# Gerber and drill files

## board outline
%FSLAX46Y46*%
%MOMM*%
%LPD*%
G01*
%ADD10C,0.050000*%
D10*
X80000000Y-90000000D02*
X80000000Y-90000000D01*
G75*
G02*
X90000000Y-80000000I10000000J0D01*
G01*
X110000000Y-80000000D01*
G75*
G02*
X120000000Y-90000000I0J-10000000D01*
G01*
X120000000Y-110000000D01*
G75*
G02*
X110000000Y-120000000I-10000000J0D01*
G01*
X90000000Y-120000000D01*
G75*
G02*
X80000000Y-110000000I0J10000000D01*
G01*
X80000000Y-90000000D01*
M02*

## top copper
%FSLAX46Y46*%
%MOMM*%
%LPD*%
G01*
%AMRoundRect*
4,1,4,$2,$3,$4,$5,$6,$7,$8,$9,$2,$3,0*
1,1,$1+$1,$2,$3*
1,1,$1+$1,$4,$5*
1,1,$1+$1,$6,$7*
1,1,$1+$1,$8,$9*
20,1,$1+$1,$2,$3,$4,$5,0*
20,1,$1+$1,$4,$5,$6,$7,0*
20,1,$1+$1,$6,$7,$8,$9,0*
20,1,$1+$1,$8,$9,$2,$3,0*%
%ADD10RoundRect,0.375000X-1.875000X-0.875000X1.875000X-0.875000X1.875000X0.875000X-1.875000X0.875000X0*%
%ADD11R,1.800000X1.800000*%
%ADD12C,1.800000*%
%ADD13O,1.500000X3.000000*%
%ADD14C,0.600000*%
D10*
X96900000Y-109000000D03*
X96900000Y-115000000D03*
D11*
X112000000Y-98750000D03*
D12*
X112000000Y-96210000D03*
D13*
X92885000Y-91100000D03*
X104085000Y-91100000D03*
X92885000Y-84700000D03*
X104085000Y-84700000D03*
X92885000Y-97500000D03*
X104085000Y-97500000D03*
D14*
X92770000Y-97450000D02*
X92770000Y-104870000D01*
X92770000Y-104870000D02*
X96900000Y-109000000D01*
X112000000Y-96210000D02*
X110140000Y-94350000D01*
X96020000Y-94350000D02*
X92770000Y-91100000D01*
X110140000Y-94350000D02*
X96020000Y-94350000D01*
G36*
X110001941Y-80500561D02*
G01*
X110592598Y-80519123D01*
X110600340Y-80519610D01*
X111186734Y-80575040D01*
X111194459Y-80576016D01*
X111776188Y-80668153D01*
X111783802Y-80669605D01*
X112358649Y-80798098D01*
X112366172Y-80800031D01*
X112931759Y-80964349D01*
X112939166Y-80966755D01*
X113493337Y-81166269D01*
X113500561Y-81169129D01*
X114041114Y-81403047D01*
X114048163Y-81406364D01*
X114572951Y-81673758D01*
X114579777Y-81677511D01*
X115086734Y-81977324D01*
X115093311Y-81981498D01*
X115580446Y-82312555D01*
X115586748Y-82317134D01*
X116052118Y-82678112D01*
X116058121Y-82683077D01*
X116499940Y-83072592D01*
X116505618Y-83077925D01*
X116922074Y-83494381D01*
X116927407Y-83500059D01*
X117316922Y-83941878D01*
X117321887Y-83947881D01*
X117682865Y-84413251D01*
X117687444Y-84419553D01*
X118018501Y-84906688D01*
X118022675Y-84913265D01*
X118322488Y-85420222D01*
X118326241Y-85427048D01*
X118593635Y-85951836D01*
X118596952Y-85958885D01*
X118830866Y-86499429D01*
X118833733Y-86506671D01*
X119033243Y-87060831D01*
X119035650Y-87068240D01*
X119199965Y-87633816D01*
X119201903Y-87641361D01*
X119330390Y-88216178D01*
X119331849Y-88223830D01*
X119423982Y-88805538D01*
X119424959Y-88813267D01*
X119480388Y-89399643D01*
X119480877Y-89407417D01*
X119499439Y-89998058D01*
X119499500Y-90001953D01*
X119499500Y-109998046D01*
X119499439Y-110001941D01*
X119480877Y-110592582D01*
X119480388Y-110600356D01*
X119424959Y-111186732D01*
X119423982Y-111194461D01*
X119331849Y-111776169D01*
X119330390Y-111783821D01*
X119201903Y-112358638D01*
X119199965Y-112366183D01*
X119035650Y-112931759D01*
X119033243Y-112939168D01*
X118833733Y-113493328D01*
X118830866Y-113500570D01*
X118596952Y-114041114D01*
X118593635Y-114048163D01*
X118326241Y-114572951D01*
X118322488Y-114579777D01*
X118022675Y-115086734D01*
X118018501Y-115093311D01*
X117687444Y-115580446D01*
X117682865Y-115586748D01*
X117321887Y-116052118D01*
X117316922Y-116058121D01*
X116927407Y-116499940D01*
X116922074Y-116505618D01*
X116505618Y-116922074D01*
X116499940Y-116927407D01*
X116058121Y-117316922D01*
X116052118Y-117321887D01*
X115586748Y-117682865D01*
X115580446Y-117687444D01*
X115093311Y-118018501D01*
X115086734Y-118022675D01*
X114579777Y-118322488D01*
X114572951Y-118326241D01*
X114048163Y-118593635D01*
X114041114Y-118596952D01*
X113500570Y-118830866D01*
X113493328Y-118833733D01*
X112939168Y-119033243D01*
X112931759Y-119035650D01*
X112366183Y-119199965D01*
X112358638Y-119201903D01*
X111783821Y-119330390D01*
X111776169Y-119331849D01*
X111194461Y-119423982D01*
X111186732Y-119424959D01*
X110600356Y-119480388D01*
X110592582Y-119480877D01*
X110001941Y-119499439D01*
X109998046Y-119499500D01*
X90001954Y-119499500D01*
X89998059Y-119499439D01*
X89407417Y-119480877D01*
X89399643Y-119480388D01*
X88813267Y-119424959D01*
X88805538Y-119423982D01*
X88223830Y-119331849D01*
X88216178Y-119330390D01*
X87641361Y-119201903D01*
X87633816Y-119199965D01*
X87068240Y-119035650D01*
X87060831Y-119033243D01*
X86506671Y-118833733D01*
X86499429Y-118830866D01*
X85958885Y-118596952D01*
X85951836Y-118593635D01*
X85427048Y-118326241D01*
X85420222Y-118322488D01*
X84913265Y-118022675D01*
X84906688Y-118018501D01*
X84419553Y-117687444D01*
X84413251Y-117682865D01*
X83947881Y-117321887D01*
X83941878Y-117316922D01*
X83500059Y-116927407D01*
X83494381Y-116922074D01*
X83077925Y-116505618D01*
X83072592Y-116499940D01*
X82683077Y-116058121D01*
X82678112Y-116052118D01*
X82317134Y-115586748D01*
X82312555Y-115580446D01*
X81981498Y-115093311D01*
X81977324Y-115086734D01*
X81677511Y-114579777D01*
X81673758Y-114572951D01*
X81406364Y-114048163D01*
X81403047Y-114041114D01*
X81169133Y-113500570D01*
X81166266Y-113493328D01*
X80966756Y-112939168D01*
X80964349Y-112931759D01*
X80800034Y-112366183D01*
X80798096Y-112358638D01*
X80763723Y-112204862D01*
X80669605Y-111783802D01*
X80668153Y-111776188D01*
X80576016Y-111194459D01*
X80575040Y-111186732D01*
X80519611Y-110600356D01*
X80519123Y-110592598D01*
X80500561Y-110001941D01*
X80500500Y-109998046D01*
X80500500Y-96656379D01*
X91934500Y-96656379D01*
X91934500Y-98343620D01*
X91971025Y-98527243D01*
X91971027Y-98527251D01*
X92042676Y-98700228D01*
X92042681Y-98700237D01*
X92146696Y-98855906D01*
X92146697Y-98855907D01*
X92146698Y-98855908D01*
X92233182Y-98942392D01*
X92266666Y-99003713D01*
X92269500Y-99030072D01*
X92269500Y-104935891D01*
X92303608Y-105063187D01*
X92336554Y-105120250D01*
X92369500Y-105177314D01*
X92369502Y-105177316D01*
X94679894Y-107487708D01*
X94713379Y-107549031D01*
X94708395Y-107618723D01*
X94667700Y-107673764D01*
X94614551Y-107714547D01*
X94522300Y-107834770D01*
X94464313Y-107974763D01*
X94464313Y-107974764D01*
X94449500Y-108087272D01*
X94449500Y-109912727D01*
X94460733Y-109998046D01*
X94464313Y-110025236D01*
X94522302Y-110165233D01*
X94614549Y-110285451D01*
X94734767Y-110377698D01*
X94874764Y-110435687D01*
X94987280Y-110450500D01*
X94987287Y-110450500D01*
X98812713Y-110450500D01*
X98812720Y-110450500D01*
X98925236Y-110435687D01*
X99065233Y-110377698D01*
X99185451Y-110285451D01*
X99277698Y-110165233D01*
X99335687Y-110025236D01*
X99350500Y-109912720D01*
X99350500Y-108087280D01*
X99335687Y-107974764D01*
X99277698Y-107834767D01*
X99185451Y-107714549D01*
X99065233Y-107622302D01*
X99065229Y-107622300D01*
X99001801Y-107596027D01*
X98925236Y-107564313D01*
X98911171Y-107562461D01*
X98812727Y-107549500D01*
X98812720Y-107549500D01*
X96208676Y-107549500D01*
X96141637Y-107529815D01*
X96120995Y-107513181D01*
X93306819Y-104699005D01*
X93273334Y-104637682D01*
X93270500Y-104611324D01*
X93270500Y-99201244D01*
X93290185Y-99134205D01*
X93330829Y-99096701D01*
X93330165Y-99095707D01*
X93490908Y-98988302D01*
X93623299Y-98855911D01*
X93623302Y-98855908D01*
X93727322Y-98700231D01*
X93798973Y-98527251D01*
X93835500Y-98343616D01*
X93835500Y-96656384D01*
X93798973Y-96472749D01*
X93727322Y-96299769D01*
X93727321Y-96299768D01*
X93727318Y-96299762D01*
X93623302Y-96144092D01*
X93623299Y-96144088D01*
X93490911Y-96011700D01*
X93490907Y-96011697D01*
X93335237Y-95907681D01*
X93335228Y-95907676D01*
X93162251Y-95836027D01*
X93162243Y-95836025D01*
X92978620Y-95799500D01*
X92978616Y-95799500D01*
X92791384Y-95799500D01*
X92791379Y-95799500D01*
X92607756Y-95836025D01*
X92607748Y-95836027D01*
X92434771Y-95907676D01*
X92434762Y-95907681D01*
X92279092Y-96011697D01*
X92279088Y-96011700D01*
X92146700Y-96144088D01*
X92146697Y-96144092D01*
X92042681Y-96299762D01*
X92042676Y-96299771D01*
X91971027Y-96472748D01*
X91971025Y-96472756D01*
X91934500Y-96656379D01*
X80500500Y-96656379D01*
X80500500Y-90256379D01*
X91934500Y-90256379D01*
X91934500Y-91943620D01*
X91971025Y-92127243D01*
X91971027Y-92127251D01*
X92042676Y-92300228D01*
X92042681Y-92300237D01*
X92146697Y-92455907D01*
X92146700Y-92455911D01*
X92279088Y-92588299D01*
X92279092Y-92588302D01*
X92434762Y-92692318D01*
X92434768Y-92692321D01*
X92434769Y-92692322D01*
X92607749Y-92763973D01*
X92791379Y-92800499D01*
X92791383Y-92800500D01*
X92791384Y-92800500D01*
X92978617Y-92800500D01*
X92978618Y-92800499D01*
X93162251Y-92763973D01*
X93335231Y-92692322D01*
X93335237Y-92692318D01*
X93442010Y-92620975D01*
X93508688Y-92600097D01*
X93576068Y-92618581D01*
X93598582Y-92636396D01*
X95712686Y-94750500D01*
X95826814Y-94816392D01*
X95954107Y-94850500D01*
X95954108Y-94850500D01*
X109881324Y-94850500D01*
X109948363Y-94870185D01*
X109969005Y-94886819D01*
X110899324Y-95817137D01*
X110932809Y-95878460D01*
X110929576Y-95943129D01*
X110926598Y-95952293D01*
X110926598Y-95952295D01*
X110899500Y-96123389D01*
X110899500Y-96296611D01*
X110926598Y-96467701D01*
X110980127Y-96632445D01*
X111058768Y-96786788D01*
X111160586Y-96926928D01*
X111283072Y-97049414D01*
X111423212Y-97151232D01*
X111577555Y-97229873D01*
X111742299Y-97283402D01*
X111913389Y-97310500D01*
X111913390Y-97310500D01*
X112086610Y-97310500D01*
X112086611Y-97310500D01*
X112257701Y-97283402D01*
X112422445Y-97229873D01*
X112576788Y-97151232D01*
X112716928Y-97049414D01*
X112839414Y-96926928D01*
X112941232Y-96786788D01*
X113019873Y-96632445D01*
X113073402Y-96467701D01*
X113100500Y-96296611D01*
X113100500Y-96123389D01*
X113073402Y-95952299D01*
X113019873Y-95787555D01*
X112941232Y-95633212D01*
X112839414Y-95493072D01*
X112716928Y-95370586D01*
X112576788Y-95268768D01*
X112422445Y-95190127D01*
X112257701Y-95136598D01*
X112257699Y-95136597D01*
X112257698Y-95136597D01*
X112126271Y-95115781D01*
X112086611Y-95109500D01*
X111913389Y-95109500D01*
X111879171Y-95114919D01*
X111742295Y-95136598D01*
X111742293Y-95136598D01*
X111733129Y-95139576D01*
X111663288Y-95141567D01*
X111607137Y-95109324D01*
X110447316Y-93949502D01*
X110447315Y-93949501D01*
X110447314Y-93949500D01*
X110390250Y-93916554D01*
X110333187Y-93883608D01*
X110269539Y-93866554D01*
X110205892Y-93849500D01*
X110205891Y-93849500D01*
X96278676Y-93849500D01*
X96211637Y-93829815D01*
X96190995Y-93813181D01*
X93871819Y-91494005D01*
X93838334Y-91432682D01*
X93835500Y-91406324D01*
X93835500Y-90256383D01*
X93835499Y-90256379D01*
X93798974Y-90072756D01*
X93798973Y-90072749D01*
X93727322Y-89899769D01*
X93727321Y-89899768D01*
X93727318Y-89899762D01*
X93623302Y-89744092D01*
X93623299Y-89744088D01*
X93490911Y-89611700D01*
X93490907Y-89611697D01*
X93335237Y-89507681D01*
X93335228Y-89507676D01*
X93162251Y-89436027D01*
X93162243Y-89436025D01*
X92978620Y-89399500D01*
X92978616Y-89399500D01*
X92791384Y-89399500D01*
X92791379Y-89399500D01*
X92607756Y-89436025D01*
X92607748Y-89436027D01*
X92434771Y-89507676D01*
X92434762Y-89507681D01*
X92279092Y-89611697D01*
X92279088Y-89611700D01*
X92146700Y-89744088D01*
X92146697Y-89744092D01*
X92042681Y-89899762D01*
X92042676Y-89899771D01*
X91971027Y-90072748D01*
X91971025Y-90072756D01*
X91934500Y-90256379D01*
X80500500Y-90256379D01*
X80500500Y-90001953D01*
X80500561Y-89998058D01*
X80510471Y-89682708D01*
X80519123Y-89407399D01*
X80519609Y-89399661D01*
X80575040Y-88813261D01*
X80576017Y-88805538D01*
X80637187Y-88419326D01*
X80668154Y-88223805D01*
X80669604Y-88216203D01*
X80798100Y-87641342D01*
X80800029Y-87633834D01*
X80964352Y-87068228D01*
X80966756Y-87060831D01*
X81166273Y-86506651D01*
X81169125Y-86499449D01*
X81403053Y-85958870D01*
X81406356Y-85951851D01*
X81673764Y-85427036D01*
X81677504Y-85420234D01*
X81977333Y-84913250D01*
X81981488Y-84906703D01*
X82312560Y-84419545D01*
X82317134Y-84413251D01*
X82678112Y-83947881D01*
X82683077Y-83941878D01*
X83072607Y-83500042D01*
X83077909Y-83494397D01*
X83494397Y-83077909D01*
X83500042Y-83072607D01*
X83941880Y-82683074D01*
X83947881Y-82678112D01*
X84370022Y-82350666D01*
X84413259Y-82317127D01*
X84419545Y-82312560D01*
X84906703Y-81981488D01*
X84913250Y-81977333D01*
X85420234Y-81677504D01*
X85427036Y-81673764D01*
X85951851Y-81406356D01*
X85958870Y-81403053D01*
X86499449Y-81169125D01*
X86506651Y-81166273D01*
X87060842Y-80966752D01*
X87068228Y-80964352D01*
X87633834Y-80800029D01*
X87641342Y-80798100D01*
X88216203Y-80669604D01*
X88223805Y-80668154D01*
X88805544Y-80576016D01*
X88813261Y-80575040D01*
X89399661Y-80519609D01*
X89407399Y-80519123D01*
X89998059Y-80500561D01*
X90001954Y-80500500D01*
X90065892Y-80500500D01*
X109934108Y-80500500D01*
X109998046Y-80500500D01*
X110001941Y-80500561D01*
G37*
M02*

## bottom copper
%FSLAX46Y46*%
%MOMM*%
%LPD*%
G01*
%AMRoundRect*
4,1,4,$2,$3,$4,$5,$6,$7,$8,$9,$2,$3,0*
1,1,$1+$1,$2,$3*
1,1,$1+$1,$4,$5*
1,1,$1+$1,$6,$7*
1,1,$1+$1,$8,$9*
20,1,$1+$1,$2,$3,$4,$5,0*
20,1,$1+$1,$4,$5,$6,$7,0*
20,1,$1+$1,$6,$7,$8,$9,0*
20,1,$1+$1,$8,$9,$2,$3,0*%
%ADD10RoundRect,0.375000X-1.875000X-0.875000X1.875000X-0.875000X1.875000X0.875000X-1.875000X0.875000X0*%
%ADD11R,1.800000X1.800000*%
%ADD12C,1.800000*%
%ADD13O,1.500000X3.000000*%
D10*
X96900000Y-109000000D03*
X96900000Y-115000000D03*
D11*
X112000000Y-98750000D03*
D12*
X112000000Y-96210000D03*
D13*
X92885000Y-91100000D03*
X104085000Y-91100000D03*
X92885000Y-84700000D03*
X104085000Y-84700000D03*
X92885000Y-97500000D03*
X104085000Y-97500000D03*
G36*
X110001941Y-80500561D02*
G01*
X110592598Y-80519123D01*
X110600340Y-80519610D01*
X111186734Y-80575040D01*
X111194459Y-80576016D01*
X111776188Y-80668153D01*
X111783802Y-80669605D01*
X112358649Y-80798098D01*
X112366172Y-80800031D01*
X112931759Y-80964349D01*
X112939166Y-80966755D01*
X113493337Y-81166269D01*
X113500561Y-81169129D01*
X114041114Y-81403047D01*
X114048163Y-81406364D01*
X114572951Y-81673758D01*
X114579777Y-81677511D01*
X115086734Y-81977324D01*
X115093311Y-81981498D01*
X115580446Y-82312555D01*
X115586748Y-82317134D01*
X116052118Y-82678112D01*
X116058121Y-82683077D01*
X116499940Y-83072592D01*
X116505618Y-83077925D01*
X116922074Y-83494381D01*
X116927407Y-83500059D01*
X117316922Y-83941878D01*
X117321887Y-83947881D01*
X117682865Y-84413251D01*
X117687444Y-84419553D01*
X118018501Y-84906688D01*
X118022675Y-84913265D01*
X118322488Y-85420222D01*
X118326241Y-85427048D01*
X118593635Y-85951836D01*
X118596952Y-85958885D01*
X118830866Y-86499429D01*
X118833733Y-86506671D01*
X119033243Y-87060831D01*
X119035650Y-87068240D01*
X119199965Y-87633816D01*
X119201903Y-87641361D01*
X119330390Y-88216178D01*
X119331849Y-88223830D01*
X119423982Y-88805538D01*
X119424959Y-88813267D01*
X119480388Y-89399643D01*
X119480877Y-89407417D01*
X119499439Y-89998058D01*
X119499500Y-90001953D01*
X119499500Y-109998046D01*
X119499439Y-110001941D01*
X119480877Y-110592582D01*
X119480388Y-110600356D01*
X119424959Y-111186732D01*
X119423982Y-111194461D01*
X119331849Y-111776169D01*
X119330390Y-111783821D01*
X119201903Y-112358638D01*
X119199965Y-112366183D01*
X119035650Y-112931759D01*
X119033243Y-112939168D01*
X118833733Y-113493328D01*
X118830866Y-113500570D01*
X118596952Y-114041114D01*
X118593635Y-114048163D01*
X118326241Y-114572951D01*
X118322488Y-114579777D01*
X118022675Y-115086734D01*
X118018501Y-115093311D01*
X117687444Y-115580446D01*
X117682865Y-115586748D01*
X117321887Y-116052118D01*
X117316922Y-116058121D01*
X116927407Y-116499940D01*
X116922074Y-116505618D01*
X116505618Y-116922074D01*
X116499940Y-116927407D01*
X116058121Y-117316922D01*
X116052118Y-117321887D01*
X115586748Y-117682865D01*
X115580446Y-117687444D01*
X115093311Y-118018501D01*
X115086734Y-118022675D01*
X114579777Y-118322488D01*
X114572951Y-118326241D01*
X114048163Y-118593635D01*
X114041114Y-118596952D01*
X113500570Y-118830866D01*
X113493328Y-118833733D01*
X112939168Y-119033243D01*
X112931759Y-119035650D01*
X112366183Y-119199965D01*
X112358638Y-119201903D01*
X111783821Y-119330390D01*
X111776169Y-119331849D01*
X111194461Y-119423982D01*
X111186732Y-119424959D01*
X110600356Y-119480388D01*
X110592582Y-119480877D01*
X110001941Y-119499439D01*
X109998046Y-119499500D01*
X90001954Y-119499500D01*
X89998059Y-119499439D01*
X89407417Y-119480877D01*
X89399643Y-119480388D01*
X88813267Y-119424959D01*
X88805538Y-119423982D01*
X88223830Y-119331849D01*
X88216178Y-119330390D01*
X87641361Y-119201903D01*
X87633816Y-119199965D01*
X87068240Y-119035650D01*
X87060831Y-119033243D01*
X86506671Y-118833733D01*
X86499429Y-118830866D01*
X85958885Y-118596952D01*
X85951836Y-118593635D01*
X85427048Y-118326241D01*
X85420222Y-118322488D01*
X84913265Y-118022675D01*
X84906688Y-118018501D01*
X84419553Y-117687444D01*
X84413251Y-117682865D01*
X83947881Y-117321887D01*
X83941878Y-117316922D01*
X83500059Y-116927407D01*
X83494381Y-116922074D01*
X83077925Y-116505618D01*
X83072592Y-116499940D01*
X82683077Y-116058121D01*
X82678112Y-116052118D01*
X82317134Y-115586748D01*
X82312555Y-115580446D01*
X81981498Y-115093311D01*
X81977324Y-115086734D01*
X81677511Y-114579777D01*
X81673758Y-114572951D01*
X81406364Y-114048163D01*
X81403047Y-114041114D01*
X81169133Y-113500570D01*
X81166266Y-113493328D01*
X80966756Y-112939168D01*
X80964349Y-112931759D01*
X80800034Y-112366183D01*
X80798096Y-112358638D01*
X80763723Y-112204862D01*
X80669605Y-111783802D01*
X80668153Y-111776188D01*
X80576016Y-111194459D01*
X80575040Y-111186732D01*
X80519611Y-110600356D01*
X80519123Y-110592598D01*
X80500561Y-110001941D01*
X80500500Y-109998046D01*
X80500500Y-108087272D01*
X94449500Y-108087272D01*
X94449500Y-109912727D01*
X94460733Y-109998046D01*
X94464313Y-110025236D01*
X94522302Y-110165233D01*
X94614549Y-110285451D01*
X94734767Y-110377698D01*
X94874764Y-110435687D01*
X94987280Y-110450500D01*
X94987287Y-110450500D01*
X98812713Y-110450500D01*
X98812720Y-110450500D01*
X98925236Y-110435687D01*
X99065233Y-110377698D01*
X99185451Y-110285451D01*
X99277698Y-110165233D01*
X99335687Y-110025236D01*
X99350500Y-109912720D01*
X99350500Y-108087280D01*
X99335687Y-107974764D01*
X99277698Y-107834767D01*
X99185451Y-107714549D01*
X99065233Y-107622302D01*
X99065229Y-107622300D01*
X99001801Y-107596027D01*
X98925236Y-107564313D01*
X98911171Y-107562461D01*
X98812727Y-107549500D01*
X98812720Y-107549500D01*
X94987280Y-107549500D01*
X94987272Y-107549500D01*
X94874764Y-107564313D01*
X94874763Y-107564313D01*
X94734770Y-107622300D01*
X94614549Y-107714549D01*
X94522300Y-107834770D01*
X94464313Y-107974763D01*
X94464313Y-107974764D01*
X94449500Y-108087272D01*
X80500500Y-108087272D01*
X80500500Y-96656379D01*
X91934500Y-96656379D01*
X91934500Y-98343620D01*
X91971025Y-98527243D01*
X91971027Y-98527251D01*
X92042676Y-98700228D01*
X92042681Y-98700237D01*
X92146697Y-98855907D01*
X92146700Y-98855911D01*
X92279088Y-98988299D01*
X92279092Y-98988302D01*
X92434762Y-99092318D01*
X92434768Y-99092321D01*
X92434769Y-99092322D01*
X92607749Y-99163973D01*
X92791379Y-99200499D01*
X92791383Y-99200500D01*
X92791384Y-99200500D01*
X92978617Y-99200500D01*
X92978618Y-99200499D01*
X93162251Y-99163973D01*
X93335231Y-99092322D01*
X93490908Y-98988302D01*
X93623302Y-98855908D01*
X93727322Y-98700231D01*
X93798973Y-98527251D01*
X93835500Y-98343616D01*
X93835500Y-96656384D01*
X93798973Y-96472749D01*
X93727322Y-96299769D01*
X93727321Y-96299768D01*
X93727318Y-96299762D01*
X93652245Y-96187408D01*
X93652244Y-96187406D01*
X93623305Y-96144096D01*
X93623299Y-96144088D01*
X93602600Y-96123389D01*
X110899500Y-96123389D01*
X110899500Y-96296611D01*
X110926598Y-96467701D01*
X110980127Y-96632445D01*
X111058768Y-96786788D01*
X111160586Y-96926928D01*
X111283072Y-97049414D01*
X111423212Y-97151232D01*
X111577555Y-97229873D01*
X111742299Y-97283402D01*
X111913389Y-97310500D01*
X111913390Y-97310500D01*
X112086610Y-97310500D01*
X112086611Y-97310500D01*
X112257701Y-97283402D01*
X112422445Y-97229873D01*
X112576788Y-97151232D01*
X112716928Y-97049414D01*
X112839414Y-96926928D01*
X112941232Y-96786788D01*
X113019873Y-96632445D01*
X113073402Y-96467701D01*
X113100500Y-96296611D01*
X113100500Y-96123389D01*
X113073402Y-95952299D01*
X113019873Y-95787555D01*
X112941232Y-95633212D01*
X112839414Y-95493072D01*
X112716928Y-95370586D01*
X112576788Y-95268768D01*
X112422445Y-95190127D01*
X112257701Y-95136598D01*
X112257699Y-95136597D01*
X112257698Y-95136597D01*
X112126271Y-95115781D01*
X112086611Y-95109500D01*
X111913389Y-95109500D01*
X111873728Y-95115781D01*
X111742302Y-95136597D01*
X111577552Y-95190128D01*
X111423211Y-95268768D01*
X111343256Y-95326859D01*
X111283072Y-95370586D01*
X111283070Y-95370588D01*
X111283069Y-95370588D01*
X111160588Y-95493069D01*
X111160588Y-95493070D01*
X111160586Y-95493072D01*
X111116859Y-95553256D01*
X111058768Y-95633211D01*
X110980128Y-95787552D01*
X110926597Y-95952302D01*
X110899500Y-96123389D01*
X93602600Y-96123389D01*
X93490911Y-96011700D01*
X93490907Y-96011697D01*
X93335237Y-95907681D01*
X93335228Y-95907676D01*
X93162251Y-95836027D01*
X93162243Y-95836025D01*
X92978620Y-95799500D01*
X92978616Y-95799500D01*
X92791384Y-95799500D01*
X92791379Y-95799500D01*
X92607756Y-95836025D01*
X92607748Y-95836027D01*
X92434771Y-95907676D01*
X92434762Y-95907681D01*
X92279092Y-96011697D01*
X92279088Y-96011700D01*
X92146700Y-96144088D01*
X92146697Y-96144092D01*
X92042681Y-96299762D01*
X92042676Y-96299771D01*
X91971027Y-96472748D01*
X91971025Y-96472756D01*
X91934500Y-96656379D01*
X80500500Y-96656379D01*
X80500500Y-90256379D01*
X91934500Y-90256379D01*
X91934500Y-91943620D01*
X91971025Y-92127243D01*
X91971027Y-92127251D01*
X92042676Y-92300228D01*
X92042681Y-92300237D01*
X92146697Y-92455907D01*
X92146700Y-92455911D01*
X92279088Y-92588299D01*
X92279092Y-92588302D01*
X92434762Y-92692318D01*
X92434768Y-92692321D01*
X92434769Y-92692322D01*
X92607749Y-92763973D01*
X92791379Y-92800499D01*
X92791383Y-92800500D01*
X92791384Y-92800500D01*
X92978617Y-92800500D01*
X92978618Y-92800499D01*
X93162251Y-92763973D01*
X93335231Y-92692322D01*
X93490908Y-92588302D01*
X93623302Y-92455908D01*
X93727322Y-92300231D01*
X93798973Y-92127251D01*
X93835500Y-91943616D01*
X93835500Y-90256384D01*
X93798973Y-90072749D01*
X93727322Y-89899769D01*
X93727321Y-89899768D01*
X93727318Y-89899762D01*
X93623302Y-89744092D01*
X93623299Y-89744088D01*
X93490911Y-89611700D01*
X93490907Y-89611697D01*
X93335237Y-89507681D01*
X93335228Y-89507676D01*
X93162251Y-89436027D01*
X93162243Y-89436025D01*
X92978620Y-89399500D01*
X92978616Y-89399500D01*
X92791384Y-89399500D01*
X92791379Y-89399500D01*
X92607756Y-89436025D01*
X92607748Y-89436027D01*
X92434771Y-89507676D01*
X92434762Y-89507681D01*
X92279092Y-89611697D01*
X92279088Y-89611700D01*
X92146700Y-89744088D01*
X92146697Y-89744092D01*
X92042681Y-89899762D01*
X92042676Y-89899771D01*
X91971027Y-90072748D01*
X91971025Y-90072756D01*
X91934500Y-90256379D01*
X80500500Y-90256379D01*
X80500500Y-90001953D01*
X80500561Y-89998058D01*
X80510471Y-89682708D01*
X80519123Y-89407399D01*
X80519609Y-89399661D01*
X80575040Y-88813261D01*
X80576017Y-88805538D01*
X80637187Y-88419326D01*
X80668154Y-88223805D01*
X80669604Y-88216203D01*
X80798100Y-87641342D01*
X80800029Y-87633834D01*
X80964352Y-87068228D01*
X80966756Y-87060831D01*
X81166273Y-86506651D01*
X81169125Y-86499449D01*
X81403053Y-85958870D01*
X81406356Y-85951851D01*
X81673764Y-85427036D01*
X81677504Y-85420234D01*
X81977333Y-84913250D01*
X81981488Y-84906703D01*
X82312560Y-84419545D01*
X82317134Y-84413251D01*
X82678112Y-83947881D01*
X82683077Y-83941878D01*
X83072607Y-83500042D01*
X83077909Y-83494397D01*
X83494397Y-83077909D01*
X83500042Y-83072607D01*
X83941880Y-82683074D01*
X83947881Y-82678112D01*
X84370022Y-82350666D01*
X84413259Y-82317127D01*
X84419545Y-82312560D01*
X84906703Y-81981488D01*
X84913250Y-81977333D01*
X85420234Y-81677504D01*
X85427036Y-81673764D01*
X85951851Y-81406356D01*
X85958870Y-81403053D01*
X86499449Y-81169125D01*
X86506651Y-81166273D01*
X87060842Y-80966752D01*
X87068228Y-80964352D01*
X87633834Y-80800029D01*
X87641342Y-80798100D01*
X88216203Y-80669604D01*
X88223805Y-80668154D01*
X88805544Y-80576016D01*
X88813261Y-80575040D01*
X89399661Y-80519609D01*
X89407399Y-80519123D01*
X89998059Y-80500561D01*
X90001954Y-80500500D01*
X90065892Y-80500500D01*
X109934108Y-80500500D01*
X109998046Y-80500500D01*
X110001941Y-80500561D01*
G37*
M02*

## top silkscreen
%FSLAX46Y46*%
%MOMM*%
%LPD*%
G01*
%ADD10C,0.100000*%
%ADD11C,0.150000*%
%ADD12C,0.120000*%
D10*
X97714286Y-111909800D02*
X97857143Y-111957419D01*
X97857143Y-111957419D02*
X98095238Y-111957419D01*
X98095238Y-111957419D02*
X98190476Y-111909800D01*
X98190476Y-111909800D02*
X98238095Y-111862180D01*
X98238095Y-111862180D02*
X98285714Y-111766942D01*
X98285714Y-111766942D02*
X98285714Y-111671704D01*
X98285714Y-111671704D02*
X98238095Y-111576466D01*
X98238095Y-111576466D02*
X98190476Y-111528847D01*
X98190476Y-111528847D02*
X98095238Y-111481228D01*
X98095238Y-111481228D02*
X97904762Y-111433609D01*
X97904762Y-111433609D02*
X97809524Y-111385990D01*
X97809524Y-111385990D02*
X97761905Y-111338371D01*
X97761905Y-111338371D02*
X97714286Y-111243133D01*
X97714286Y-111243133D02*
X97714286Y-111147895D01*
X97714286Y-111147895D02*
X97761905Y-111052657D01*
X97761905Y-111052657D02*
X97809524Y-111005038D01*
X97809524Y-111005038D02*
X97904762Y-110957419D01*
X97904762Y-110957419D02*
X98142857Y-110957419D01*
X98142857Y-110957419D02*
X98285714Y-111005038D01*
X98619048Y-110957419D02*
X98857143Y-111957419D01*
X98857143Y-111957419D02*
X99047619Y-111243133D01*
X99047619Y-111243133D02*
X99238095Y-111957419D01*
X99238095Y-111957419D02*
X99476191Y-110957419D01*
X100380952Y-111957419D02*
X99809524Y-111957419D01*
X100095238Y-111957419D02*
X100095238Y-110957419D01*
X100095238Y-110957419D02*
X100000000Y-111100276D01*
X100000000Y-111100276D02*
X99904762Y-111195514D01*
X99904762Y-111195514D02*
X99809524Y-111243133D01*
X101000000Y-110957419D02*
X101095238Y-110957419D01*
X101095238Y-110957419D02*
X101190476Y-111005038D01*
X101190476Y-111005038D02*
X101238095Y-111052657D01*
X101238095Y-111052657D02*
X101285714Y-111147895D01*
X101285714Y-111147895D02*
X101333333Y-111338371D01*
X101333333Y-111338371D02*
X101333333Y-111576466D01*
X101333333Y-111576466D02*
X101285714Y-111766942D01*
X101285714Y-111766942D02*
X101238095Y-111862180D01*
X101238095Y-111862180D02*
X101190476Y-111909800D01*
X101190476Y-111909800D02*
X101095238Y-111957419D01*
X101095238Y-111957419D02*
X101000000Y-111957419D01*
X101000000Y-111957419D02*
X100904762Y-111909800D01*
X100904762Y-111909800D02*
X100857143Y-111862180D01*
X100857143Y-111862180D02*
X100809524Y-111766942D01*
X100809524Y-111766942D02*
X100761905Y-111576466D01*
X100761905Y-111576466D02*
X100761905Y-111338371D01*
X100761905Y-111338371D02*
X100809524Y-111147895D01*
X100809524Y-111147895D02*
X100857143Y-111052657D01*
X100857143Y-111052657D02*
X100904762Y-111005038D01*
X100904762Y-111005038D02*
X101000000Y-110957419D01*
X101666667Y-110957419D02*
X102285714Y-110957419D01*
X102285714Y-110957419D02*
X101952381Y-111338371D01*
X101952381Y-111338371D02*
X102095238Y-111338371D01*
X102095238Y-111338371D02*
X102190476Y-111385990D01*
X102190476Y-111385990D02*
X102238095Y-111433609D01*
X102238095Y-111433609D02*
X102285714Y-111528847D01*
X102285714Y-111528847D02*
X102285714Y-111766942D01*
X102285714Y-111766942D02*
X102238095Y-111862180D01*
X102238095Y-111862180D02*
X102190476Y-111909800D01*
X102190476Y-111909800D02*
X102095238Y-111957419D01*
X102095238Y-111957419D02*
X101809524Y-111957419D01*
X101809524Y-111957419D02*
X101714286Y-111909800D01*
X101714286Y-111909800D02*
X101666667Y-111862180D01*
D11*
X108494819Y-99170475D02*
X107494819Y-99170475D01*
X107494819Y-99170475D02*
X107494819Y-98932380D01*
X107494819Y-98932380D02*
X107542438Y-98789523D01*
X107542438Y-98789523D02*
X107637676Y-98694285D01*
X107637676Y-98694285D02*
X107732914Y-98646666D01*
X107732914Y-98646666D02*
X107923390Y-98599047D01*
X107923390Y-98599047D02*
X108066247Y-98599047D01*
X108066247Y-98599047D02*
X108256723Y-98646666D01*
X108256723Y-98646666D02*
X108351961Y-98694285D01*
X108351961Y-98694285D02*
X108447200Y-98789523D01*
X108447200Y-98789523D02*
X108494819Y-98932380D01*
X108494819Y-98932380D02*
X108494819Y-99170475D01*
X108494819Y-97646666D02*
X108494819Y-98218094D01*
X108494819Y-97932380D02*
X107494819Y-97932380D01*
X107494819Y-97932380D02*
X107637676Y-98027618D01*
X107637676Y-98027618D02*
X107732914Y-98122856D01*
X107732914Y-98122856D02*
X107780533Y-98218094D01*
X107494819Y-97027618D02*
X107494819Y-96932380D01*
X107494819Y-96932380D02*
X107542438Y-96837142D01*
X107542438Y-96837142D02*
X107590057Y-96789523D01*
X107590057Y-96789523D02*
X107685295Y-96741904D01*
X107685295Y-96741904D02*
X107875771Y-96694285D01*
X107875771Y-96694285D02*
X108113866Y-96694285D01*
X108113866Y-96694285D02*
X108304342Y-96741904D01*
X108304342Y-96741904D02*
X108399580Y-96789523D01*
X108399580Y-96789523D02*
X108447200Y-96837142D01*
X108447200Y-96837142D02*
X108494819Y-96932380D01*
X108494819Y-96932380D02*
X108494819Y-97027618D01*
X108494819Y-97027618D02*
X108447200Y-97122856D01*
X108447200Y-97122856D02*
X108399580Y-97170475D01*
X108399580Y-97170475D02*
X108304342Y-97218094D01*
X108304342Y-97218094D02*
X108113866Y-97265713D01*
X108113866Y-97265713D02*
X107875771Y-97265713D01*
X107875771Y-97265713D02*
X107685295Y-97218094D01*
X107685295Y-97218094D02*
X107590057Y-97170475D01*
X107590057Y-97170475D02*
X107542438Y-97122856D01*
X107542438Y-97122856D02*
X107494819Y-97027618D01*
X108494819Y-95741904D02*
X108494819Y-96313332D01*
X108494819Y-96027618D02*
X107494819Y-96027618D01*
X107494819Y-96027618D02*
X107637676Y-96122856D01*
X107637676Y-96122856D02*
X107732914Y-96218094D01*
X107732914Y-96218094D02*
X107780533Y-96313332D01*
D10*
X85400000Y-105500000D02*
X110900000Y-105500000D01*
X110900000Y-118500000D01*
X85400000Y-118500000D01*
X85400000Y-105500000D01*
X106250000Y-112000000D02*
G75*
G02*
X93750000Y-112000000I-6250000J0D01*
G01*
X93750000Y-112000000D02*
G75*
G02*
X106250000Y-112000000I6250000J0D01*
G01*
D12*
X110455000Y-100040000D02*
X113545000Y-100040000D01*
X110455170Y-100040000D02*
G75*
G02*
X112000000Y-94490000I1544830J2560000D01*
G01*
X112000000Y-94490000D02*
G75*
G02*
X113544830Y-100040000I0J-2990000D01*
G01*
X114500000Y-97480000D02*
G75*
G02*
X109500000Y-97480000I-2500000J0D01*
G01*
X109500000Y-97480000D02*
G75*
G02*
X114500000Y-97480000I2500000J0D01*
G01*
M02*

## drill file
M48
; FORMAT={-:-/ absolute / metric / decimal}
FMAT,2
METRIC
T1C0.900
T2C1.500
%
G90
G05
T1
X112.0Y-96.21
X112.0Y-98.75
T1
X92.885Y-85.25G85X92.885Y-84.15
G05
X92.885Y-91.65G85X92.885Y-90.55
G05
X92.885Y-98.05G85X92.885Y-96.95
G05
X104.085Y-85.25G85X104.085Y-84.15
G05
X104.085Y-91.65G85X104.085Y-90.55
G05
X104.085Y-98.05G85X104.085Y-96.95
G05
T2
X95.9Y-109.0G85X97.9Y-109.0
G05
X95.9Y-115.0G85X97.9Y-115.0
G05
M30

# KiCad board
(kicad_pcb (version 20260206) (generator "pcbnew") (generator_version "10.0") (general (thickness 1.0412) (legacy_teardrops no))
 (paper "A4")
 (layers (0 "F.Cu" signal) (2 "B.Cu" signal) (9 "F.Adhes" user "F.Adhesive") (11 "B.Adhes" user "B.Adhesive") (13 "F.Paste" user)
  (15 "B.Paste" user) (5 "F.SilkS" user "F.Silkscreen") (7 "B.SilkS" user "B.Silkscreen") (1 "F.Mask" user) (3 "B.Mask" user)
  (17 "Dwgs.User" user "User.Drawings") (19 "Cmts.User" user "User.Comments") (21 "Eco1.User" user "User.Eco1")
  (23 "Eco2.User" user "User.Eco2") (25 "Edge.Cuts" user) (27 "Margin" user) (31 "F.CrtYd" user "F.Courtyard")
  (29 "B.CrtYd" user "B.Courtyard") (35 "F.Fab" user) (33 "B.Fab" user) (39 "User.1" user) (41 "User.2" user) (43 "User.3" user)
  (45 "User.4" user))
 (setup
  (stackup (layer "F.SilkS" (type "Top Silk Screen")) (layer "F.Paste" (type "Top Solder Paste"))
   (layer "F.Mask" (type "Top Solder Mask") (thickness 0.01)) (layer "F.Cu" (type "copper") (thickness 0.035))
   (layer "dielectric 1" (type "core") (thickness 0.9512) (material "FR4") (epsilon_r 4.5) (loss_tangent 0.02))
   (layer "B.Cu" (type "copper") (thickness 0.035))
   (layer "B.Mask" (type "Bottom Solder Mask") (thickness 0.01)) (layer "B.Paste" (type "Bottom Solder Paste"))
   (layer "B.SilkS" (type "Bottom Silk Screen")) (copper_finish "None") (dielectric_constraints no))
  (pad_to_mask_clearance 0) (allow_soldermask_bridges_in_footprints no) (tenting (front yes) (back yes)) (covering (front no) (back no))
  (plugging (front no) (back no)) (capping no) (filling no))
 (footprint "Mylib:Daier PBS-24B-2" (layer "F.Cu") (at 100 112)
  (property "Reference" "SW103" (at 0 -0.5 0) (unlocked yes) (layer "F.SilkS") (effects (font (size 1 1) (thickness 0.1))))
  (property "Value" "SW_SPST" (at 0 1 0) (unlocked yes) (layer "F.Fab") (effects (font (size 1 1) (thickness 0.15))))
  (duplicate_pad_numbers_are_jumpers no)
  (fp_rect (start -14.6 -6.5) (end 10.9 6.5) (stroke (width 0.1) (type solid)) (fill no) (layer "F.SilkS"))
  (fp_circle (center 0 0) (end 6.25 0) (stroke (width 0.1) (type solid)) (fill no) (layer "F.SilkS"))
  (pad "1" thru_hole roundrect (at -3.1 -3) (size 4.5 2.5) (drill oval 3.5 1.5) (layers "*.Cu" "*.Mask") (remove_unused_layers no)
   (roundrect_rratio 0.15) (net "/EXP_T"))
  (pad "2" thru_hole roundrect (at -3.1 3) (size 4.5 2.5) (drill oval 3.5 1.5) (layers "*.Cu" "*.Mask") (remove_unused_layers no)
   (roundrect_rratio 0.15) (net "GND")))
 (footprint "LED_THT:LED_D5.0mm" (layer "F.Cu") (at 112 98.75 90)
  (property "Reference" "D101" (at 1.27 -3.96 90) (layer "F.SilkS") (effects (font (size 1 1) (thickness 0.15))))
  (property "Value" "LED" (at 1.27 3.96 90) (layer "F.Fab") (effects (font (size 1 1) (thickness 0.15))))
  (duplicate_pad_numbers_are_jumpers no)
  (fp_line (start -1.29 -1.545) (end -1.29 1.545) (stroke (width 0.12) (type solid)) (layer "F.SilkS"))
  (fp_arc (start -1.29 -1.54483) (mid 2.071779 -2.880495) (end 4.26 0) (stroke (width 0.12) (type solid)) (layer "F.SilkS"))
  (fp_arc (start 4.26 0) (mid 2.071779 2.880495) (end -1.29 1.54483) (stroke (width 0.12) (type solid)) (layer "F.SilkS"))
  (fp_circle (center 1.27 0) (end 3.77 0) (stroke (width 0.12) (type solid)) (fill no) (layer "F.SilkS"))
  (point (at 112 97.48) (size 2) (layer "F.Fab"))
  (pad "1" thru_hole rect (at 0 0 90) (size 1.8 1.8) (drill 0.9) (layers "*.Cu" "*.Mask") (remove_unused_layers no) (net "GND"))
  (pad "2" thru_hole circle (at 2.54 0 90) (size 1.8 1.8) (drill 0.9) (layers "*.Cu" "*.Mask") (remove_unused_layers no) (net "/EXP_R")))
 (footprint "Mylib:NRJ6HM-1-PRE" (layer "F.Cu") (at 100 80 90)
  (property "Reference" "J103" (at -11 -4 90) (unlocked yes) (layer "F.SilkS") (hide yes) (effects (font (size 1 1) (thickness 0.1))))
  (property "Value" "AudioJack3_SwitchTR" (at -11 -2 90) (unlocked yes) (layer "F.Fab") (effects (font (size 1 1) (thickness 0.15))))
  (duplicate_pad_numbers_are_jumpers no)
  (pad "R" thru_hole oval (at -11.1 -7.115 90) (size 3 1.5) (drill oval 2 0.9) (layers "*.Cu" "*.Mask") (remove_unused_layers no)
   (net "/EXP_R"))
  (pad "RN" thru_hole oval (at -11.1 4.085 90) (size 3 1.5) (drill oval 2 0.9) (layers "*.Cu" "*.Mask") (remove_unused_layers no)
   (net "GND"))
  (pad "S" thru_hole oval (at -4.7 -7.115 90) (size 3 1.5) (drill oval 2 0.9) (layers "*.Cu" "*.Mask") (remove_unused_layers no) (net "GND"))
  (pad "S" thru_hole oval (at -4.7 4.085 90) (size 3 1.5) (drill oval 2 0.9) (layers "*.Cu" "*.Mask") (remove_unused_layers no) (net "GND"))
  (pad "T" thru_hole oval (at -17.5 -7.115 90) (size 3 1.5) (drill oval 2 0.9) (layers "*.Cu" "*.Mask") (remove_unused_layers no)
   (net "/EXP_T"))
  (pad "TN" thru_hole oval (at -17.5 4.085 90) (size 3 1.5) (drill oval 2 0.9) (layers "*.Cu" "*.Mask") (remove_unused_layers no)
   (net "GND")))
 (gr_rect (start 80 80) (end 120 120) (radius 10) (stroke (width 0.05) (type solid)) (fill no) (layer "Edge.Cuts"))
 (segment (start 92.77 97.45) (end 92.77 104.87) (width 0.6) (layer "F.Cu") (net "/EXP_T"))
 (segment (start 92.77 104.87) (end 96.9 109) (width 0.6) (layer "F.Cu") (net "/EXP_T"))
 (segment (start 112 96.21) (end 110.14 94.35) (width 0.6) (layer "F.Cu") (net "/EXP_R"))
 (segment (start 96.02 94.35) (end 92.77 91.1) (width 0.6) (layer "F.Cu") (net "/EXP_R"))
 (segment (start 110.14 94.35) (end 96.02 94.35) (width 0.6) (layer "F.Cu") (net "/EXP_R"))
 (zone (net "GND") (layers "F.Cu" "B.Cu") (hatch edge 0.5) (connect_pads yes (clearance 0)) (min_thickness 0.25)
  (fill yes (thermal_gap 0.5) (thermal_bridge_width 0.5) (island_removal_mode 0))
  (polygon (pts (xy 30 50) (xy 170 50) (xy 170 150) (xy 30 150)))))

